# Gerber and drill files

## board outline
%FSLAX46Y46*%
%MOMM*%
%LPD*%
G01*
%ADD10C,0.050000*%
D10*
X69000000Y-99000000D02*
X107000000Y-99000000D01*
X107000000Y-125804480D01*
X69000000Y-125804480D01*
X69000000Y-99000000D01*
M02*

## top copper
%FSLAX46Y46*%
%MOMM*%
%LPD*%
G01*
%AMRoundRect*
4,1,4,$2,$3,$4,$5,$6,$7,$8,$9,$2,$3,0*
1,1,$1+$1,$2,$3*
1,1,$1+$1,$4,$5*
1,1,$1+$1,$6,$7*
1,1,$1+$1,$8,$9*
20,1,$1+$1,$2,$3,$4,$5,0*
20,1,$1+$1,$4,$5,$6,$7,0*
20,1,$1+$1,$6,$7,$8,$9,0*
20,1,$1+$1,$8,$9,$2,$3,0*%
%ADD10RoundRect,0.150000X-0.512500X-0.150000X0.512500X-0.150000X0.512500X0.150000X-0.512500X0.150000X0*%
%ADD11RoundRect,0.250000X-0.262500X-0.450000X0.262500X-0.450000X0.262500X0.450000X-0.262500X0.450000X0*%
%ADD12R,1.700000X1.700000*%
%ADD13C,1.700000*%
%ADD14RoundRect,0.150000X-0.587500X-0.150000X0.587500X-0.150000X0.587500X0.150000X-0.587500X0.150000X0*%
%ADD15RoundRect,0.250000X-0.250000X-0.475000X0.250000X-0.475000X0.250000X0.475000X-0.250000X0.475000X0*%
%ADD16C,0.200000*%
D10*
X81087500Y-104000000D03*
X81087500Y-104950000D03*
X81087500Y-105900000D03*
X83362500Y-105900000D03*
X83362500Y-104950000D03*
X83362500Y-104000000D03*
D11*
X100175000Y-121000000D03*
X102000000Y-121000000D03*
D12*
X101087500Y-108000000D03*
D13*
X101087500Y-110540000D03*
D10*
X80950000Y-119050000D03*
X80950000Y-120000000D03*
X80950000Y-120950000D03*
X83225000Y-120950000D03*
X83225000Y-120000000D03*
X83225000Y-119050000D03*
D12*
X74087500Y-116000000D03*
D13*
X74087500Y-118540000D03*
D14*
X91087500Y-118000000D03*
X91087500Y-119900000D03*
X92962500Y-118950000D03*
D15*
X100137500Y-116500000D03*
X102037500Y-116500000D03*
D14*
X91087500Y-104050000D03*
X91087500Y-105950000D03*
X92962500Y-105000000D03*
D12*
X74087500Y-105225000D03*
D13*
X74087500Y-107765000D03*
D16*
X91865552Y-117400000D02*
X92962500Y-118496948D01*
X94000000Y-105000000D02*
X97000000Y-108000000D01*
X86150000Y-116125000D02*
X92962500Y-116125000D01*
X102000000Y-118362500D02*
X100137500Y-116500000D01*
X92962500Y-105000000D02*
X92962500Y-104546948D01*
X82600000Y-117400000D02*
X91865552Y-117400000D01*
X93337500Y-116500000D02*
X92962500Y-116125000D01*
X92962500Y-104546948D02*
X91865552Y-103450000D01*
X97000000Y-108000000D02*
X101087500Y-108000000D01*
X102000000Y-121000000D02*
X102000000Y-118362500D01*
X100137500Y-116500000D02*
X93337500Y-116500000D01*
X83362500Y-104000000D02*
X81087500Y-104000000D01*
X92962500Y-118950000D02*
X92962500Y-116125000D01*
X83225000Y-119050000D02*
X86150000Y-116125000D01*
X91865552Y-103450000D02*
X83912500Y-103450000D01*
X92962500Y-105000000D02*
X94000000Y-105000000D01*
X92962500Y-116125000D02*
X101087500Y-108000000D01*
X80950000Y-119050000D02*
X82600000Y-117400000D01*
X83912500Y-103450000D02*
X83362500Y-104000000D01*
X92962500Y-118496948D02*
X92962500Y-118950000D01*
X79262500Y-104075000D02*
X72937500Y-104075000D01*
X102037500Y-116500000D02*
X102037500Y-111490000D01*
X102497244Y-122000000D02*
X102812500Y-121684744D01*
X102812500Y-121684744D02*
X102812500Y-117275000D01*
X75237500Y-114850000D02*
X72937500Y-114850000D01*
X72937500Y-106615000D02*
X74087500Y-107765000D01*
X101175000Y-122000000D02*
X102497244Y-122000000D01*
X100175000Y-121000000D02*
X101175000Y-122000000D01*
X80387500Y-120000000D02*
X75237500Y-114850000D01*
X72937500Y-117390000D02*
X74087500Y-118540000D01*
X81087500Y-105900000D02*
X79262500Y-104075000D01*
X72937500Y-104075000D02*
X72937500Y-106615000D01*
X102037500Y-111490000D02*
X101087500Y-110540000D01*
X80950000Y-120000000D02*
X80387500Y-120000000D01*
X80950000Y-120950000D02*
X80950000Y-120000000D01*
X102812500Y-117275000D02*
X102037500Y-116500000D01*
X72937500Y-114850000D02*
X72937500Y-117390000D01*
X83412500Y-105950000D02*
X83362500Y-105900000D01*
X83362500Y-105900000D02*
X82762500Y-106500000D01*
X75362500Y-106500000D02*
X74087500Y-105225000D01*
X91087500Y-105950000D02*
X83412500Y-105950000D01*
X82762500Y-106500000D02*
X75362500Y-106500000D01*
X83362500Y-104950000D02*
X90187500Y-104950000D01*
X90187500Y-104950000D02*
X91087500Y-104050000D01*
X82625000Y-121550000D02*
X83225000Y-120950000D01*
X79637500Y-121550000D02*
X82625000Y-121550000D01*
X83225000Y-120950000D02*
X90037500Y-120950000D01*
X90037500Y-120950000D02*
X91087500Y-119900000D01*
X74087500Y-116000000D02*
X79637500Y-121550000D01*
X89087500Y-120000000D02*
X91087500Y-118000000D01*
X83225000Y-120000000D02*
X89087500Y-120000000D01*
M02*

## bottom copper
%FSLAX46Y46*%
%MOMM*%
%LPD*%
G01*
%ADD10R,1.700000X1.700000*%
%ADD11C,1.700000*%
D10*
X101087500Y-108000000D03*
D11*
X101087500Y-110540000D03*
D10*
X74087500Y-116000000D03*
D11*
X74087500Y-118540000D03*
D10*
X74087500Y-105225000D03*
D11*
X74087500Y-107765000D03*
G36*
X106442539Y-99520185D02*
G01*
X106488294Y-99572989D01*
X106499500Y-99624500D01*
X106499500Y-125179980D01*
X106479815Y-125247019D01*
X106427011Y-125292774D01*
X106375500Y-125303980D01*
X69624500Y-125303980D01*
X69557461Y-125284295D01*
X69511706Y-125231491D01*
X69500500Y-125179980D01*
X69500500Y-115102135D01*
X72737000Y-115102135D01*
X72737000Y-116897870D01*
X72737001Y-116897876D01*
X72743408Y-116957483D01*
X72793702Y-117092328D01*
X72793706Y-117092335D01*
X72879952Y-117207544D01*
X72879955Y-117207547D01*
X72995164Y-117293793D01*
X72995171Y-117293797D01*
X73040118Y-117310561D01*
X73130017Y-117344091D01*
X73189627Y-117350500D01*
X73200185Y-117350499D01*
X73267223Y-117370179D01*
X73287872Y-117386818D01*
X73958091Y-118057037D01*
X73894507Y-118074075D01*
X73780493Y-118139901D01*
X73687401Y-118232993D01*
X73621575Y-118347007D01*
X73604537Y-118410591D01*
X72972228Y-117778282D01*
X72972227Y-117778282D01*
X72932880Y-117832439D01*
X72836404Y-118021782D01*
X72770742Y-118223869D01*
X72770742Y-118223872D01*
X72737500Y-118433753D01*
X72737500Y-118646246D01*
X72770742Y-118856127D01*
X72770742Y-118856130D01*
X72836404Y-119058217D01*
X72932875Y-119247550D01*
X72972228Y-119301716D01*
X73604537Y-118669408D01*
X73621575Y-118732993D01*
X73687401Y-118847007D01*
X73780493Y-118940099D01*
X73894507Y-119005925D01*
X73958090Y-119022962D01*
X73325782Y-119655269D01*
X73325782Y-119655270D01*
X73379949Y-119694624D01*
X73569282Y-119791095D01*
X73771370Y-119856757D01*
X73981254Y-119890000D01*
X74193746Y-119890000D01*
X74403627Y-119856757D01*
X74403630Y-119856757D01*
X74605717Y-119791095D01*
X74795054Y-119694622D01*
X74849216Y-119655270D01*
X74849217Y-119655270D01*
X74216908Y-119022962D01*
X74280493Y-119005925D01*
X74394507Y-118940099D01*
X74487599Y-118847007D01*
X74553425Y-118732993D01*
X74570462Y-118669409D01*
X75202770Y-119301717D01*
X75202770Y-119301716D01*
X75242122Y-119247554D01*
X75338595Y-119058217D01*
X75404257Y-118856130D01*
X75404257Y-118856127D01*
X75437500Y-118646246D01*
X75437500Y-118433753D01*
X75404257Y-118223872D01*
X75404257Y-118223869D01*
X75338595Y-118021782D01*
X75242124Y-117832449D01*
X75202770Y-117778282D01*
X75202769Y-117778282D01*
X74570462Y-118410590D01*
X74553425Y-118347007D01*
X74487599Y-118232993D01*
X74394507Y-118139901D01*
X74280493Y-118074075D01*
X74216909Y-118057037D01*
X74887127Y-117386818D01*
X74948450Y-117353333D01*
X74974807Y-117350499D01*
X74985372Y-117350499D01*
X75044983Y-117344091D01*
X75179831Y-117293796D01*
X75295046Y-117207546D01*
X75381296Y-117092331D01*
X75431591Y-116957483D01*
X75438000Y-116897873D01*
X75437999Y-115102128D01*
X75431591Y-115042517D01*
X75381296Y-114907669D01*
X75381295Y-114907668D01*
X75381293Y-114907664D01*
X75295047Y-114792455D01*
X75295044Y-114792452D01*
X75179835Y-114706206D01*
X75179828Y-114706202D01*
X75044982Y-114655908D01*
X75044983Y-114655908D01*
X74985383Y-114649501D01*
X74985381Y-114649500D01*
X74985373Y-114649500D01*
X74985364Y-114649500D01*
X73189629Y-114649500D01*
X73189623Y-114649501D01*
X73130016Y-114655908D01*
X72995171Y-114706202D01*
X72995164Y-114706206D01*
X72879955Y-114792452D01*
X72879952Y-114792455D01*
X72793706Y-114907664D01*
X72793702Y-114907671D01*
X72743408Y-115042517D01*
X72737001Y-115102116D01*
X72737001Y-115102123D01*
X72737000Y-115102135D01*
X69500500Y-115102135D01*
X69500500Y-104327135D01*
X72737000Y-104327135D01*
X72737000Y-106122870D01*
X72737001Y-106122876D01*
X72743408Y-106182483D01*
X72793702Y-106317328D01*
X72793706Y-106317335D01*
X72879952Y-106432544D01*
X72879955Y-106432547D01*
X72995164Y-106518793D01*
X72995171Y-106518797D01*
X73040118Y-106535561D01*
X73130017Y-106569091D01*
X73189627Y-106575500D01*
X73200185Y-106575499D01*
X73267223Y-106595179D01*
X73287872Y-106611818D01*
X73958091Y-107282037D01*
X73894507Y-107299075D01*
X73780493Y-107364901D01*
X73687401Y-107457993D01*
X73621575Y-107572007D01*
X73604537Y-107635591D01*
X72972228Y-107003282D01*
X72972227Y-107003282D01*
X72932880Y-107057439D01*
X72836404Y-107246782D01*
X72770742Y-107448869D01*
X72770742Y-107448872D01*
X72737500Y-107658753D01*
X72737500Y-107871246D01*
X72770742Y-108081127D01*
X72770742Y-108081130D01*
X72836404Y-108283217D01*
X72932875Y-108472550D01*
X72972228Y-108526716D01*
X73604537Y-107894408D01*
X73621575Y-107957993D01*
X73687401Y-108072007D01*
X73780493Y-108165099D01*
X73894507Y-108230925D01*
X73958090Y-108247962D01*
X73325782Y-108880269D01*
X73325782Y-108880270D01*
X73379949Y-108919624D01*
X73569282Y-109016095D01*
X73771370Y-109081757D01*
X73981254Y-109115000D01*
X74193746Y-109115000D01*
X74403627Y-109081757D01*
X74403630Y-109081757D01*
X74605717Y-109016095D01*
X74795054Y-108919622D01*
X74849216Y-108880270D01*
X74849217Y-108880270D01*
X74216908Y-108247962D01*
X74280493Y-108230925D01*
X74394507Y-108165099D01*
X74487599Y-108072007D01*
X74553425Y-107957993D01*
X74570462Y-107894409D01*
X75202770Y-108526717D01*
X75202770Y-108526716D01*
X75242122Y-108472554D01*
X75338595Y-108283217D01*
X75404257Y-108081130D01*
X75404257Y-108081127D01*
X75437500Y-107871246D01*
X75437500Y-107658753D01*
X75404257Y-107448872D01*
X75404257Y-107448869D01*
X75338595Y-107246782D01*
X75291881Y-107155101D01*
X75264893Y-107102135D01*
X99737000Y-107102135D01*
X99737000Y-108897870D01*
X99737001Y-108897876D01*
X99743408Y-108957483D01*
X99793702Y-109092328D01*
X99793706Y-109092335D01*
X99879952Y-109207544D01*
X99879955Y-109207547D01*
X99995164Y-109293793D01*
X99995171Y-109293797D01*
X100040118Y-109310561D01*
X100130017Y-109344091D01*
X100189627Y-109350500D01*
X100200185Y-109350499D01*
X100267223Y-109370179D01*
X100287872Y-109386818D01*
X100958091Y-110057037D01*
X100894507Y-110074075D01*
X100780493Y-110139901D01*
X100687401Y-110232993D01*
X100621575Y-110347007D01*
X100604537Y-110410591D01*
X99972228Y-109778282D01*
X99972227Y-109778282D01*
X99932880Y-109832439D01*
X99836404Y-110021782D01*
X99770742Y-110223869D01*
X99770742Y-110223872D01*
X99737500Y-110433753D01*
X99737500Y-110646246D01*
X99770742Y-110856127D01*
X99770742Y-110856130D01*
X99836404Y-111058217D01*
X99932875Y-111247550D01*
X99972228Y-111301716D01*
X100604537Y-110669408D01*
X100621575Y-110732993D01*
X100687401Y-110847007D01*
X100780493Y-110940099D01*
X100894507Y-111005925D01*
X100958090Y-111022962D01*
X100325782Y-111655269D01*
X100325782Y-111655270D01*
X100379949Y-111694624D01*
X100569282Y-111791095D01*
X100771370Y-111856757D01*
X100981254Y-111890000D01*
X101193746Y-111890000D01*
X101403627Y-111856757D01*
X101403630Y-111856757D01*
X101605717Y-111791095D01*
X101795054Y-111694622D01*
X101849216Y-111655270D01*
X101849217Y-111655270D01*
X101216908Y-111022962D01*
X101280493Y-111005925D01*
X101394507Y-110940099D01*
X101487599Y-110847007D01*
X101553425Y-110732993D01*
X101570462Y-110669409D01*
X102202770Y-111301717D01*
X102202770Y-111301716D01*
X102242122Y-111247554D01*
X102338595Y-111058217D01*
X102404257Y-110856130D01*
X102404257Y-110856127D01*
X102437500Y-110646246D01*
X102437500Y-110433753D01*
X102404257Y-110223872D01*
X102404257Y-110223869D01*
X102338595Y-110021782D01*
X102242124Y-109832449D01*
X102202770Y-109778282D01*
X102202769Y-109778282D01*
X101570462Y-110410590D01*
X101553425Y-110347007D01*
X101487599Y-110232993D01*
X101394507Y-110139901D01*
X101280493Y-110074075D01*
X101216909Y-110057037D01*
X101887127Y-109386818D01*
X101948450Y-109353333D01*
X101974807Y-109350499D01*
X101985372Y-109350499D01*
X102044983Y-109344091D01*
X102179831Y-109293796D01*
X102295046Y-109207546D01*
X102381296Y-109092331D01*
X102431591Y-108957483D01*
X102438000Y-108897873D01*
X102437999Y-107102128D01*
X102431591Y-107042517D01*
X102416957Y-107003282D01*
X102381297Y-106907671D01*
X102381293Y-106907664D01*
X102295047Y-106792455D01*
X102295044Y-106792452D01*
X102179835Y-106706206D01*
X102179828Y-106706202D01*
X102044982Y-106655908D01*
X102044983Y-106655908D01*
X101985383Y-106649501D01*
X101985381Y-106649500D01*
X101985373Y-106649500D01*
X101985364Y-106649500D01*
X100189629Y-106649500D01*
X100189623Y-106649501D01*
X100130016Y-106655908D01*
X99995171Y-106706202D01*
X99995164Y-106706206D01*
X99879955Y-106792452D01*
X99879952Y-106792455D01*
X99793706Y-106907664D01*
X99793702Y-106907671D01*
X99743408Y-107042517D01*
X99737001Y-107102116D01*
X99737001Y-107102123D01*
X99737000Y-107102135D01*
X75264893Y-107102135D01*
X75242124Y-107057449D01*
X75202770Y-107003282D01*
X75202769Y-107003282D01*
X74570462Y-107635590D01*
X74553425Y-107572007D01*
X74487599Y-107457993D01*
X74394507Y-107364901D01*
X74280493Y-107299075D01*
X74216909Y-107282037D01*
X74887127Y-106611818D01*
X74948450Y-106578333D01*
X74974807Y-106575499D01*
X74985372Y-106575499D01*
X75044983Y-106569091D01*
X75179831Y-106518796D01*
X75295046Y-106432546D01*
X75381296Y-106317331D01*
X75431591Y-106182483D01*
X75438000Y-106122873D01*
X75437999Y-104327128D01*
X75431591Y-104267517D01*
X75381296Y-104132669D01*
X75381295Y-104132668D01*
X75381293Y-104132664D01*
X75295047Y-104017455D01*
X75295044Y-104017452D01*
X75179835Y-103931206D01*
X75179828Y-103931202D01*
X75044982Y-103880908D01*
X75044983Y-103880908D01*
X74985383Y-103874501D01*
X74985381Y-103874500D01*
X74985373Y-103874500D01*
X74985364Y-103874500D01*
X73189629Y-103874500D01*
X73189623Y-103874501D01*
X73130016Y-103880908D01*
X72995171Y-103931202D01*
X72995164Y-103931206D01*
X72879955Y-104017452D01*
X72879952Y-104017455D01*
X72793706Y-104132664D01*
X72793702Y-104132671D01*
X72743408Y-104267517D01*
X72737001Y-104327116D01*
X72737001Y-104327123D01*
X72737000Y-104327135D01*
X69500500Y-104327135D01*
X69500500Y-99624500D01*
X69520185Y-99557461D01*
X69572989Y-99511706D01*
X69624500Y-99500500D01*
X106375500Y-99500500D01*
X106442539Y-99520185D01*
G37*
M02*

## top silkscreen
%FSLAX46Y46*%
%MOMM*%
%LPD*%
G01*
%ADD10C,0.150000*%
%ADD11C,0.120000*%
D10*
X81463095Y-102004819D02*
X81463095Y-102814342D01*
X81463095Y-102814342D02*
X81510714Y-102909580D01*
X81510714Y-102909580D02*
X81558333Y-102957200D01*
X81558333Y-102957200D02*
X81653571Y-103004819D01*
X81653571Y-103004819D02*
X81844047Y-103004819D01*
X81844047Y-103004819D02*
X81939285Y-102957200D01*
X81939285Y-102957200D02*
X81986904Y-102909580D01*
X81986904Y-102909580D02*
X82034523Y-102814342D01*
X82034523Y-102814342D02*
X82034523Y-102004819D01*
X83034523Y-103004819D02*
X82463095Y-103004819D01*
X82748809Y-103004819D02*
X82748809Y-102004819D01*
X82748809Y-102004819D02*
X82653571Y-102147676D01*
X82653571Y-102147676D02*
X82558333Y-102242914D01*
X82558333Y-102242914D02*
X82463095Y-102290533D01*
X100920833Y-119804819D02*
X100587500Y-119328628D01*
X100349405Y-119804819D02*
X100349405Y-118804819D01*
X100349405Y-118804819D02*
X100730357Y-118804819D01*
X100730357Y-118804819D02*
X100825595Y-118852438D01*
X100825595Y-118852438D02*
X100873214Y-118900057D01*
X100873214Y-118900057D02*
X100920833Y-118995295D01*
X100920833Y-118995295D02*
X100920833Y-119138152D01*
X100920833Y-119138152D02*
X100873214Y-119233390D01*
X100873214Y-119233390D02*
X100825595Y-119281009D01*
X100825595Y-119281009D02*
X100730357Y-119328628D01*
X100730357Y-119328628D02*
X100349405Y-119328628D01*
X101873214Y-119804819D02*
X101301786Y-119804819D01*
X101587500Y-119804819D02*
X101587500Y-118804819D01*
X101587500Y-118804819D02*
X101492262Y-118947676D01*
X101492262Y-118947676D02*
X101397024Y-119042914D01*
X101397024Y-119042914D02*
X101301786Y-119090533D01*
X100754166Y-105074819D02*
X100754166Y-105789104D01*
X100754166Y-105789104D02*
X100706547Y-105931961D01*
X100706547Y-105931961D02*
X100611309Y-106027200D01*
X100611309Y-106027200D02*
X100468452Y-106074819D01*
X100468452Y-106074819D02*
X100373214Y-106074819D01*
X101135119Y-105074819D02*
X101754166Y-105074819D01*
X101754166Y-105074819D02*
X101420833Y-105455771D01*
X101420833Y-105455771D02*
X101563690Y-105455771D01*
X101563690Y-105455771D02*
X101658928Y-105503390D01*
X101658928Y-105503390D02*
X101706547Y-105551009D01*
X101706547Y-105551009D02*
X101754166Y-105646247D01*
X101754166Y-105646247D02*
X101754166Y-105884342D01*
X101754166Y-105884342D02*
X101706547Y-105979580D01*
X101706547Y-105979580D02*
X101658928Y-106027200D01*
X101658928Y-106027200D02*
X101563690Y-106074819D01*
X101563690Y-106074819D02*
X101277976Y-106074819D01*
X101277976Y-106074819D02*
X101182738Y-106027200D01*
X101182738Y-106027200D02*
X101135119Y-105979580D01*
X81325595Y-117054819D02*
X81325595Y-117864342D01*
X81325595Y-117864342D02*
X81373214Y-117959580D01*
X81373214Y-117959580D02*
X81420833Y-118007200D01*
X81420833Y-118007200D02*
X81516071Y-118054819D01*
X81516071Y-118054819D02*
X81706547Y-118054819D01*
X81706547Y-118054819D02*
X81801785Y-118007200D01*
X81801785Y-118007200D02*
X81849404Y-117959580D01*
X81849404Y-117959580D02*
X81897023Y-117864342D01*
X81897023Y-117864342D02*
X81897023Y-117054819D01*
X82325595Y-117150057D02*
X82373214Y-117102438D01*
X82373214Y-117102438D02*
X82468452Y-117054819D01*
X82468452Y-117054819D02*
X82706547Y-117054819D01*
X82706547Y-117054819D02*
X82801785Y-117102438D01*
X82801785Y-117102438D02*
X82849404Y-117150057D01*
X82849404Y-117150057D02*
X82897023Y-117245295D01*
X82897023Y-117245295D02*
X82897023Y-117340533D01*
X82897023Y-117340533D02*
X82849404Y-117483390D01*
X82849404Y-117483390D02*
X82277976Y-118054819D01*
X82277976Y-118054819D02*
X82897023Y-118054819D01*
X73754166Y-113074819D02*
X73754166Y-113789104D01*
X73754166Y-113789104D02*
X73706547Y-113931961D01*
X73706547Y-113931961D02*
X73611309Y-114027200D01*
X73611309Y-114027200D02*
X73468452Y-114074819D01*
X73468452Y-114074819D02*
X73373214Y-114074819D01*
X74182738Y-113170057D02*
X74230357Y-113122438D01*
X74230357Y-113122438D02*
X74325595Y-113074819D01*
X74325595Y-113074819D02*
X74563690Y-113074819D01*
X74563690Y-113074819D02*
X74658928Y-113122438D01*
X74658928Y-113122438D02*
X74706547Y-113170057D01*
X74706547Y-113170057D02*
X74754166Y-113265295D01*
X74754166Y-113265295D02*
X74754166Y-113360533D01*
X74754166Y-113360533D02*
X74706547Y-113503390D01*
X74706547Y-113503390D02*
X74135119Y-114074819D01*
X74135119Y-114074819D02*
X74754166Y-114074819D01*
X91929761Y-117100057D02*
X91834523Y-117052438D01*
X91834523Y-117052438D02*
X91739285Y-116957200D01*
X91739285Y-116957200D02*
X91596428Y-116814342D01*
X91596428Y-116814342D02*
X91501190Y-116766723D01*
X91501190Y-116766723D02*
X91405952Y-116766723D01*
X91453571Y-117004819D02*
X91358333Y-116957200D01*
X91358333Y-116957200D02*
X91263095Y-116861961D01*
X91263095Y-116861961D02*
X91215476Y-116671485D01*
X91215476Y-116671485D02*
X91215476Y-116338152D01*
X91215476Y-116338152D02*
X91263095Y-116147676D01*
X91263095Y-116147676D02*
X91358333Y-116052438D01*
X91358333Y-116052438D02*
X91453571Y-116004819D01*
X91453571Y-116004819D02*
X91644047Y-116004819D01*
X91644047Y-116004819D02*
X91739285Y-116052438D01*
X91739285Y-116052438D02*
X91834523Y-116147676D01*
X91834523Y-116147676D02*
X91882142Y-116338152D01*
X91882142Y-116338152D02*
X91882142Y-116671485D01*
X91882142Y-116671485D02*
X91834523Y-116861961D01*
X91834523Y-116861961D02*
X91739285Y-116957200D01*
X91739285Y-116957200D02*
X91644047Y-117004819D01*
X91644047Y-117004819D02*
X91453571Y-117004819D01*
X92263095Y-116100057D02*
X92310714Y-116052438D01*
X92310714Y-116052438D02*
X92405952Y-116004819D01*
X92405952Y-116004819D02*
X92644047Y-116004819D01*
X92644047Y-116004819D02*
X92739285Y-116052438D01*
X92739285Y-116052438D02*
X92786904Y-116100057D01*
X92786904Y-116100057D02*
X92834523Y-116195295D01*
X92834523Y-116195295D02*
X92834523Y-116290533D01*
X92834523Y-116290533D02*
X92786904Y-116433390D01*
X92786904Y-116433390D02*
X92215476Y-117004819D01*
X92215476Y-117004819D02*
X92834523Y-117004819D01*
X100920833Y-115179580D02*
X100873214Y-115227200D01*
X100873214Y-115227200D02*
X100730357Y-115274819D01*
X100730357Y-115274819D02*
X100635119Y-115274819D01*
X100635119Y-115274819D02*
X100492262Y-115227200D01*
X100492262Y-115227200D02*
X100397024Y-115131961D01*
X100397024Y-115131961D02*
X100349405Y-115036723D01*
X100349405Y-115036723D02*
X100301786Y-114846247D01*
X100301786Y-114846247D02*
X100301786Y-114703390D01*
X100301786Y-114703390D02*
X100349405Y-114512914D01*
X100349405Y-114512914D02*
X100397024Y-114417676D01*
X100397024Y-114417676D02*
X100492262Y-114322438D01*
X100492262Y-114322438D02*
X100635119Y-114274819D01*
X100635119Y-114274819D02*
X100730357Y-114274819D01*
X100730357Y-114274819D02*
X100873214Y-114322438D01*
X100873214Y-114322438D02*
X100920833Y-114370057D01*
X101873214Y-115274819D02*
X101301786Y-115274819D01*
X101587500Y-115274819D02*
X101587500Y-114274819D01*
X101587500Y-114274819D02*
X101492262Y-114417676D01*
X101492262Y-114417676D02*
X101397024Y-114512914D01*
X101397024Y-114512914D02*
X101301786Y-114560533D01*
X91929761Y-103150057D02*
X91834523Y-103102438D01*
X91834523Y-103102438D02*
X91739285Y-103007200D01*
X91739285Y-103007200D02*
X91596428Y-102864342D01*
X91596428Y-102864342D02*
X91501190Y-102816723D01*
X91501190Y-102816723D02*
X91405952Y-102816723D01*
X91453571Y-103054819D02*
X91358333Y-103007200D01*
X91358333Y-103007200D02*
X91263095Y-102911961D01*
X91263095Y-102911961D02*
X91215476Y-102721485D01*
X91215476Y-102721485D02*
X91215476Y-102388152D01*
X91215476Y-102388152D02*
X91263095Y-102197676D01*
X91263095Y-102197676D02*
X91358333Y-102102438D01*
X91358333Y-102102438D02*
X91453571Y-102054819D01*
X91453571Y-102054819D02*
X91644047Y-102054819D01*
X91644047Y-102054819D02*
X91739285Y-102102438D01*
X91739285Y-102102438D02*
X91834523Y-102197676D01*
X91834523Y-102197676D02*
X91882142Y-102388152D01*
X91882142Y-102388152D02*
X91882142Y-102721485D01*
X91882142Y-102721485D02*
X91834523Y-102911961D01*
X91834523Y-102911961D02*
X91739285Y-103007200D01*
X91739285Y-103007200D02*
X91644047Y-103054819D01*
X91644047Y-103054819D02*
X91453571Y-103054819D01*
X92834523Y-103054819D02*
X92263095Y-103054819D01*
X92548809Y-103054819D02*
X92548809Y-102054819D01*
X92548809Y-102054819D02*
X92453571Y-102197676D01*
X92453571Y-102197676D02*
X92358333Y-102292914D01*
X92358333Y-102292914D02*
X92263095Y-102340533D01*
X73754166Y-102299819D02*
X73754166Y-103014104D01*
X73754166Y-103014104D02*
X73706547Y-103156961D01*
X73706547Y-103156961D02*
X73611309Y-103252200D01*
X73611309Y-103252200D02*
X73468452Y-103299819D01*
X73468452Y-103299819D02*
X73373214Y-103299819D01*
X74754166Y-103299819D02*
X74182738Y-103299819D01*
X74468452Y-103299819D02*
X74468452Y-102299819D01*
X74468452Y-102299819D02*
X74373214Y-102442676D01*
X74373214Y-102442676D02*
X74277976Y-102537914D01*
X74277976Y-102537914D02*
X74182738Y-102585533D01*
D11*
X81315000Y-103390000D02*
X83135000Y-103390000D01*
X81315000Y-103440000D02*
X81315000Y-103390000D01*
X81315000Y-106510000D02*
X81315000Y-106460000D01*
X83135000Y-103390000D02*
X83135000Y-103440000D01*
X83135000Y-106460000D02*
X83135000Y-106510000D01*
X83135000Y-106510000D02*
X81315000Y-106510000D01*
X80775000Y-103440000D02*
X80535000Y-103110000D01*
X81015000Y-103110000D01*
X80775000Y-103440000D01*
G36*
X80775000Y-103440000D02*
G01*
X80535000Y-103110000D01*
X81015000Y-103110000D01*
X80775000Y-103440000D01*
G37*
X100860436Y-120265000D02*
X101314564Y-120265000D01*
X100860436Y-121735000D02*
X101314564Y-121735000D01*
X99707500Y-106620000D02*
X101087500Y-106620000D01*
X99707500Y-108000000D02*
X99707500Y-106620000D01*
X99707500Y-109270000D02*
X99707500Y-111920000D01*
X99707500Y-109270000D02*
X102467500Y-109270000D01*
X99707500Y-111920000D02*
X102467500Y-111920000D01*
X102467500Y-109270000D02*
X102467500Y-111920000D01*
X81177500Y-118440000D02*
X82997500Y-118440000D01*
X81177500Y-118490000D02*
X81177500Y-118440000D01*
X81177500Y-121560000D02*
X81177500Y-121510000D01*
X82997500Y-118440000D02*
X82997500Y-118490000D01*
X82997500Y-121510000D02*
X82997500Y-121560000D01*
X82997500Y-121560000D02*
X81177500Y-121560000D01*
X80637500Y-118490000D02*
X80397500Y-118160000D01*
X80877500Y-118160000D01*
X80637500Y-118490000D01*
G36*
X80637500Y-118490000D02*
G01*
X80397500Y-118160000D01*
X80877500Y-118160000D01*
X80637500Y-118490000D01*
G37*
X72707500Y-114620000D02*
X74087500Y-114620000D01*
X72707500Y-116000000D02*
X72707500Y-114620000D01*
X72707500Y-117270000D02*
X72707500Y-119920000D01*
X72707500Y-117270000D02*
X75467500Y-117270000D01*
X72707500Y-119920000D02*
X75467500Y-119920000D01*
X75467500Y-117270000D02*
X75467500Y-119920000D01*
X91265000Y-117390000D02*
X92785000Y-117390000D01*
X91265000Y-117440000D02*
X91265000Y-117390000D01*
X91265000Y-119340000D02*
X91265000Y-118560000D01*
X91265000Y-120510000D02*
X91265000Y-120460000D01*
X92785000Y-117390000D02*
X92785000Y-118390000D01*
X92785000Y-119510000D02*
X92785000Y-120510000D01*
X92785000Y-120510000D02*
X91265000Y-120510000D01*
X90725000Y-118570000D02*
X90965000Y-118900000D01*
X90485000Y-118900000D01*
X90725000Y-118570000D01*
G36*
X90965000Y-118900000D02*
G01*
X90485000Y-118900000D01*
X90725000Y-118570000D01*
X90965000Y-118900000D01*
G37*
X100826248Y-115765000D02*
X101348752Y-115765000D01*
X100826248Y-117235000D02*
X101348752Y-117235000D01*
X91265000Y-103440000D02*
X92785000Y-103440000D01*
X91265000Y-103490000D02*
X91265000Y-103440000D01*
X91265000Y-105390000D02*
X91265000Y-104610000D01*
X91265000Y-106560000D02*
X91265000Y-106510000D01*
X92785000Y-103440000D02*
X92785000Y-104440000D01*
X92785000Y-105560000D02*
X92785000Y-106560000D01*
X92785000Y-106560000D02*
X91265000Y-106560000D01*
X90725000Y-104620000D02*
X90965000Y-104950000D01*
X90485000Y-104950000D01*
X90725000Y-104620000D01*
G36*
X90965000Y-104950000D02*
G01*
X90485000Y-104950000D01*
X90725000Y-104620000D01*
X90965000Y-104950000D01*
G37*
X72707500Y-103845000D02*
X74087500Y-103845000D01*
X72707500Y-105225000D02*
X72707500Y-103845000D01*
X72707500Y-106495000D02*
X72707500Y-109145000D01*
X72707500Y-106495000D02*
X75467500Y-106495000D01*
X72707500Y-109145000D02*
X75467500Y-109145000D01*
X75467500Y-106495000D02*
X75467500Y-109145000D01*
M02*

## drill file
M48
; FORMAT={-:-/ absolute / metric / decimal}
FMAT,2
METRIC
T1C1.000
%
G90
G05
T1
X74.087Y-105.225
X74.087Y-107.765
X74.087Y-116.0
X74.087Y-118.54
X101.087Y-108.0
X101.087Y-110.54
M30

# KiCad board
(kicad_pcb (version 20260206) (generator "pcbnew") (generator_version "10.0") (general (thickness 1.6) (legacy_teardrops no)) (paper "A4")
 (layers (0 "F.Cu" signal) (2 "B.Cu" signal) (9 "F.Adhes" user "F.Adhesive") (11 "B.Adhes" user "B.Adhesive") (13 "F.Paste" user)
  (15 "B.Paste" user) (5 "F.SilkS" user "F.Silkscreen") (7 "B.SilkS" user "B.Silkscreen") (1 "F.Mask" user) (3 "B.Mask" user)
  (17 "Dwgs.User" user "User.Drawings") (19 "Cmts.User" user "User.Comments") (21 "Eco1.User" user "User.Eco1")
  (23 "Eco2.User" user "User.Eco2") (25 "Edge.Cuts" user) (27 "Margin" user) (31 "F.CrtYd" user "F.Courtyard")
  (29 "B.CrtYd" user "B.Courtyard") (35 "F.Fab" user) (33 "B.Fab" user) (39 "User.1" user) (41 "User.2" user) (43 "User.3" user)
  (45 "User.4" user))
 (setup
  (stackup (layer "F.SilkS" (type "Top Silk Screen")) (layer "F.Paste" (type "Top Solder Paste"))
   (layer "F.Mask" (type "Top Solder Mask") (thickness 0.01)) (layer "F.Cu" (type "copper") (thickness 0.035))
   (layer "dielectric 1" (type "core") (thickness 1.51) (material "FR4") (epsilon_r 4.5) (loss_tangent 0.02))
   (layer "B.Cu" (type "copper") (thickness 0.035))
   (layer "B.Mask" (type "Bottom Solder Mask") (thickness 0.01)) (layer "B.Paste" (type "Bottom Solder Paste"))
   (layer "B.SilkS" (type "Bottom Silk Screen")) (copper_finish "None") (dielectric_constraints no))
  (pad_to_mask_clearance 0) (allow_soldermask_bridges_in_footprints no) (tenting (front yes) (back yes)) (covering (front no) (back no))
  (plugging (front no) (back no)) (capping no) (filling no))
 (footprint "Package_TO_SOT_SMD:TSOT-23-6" (layer "F.Cu") (at 82.225 104.95)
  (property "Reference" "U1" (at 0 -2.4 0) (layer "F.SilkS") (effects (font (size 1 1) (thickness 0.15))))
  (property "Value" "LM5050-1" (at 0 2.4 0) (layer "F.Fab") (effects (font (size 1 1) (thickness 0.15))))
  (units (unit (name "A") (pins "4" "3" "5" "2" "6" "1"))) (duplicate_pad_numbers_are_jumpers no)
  (fp_line (start -0.91 -1.56) (end 0.91 -1.56) (stroke (width 0.12) (type solid)) (layer "F.SilkS"))
  (fp_line (start -0.91 -1.51) (end -0.91 -1.56) (stroke (width 0.12) (type solid)) (layer "F.SilkS"))
  (fp_line (start -0.91 1.56) (end -0.91 1.51) (stroke (width 0.12) (type solid)) (layer "F.SilkS"))
  (fp_line (start 0.91 -1.56) (end 0.91 -1.51) (stroke (width 0.12) (type solid)) (layer "F.SilkS"))
  (fp_line (start 0.91 1.51) (end 0.91 1.56) (stroke (width 0.12) (type solid)) (layer "F.SilkS"))
  (fp_line (start 0.91 1.56) (end -0.91 1.56) (stroke (width 0.12) (type solid)) (layer "F.SilkS"))
  (fp_poly (pts (xy -1.45 -1.51) (xy -1.69 -1.84) (xy -1.21 -1.84)) (stroke (width 0.12) (type solid)) (fill yes) (layer "F.SilkS"))
  (pad "1" smd roundrect (at -1.1375 -0.95) (size 1.325 0.6) (layers "F.Cu" "F.Mask" "F.Paste") (roundrect_rratio 0.25)
   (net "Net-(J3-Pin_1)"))
  (pad "2" smd roundrect (at -1.1375 0) (size 1.325 0.6) (layers "F.Cu" "F.Mask" "F.Paste") (roundrect_rratio 0.25) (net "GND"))
  (pad "3" smd roundrect (at -1.1375 0.95) (size 1.325 0.6) (layers "F.Cu" "F.Mask" "F.Paste") (roundrect_rratio 0.25) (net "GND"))
  (pad "4" smd roundrect (at 1.1375 0.95) (size 1.325 0.6) (layers "F.Cu" "F.Mask" "F.Paste") (roundrect_rratio 0.25) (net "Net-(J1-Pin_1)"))
  (pad "5" smd roundrect (at 1.1375 0) (size 1.325 0.6) (layers "F.Cu" "F.Mask" "F.Paste") (roundrect_rratio 0.25) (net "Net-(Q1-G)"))
  (pad "6" smd roundrect (at 1.1375 -0.95) (size 1.325 0.6) (layers "F.Cu" "F.Mask" "F.Paste") (roundrect_rratio 0.25)
   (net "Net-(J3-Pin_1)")))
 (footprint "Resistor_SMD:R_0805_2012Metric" (layer "F.Cu") (at 101.0875 121)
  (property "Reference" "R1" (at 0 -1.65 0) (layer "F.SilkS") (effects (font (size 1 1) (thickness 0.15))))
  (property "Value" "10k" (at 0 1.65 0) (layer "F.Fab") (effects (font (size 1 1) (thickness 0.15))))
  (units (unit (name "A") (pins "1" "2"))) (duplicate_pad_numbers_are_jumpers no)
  (fp_line (start -0.227064 -0.735) (end 0.227064 -0.735) (stroke (width 0.12) (type solid)) (layer "F.SilkS"))
  (fp_line (start -0.227064 0.735) (end 0.227064 0.735) (stroke (width 0.12) (type solid)) (layer "F.SilkS"))
  (pad "1" smd roundrect (at -0.9125 0) (size 1.025 1.4) (layers "F.Cu" "F.Mask" "F.Paste") (roundrect_rratio 0.243902) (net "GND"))
  (pad "2" smd roundrect (at 0.9125 0) (size 1.025 1.4) (layers "F.Cu" "F.Mask" "F.Paste") (roundrect_rratio 0.243902)
   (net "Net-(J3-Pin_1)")))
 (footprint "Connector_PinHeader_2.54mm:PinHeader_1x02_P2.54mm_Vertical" (layer "F.Cu") (at 101.0875 108)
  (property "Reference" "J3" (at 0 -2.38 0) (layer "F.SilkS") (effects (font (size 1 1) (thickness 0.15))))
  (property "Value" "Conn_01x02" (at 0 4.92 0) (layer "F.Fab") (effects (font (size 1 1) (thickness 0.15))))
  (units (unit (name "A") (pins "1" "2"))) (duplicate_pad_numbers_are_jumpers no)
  (fp_line (start -1.38 -1.38) (end 0 -1.38) (stroke (width 0.12) (type solid)) (layer "F.SilkS"))
  (fp_line (start -1.38 0) (end -1.38 -1.38) (stroke (width 0.12) (type solid)) (layer "F.SilkS"))
  (fp_line (start -1.38 1.27) (end -1.38 3.92) (stroke (width 0.12) (type solid)) (layer "F.SilkS"))
  (fp_line (start -1.38 1.27) (end 1.38 1.27) (stroke (width 0.12) (type solid)) (layer "F.SilkS"))
  (fp_line (start -1.38 3.92) (end 1.38 3.92) (stroke (width 0.12) (type solid)) (layer "F.SilkS"))
  (fp_line (start 1.38 1.27) (end 1.38 3.92) (stroke (width 0.12) (type solid)) (layer "F.SilkS"))
  (pad "1" thru_hole rect (at 0 0) (size 1.7 1.7) (drill 1) (layers "*.Cu" "*.Mask") (remove_unused_layers no) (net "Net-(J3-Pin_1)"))
  (pad "2" thru_hole circle (at 0 2.54) (size 1.7 1.7) (drill 1) (layers "*.Cu" "*.Mask") (remove_unused_layers no) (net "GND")))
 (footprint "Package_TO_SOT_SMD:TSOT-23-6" (layer "F.Cu") (at 82.0875 120)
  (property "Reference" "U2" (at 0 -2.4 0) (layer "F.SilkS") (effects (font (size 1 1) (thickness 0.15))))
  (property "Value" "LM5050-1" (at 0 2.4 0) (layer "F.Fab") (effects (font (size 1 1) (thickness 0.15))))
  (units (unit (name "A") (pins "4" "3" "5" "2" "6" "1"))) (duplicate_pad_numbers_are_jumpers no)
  (fp_line (start -0.91 -1.56) (end 0.91 -1.56) (stroke (width 0.12) (type solid)) (layer "F.SilkS"))
  (fp_line (start -0.91 -1.51) (end -0.91 -1.56) (stroke (width 0.12) (type solid)) (layer "F.SilkS"))
  (fp_line (start -0.91 1.56) (end -0.91 1.51) (stroke (width 0.12) (type solid)) (layer "F.SilkS"))
  (fp_line (start 0.91 -1.56) (end 0.91 -1.51) (stroke (width 0.12) (type solid)) (layer "F.SilkS"))
  (fp_line (start 0.91 1.51) (end 0.91 1.56) (stroke (width 0.12) (type solid)) (layer "F.SilkS"))
  (fp_line (start 0.91 1.56) (end -0.91 1.56) (stroke (width 0.12) (type solid)) (layer "F.SilkS"))
  (fp_poly (pts (xy -1.45 -1.51) (xy -1.69 -1.84) (xy -1.21 -1.84)) (stroke (width 0.12) (type solid)) (fill yes) (layer "F.SilkS"))
  (pad "1" smd roundrect (at -1.1375 -0.95) (size 1.325 0.6) (layers "F.Cu" "F.Mask" "F.Paste") (roundrect_rratio 0.25)
   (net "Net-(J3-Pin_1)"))
  (pad "2" smd roundrect (at -1.1375 0) (size 1.325 0.6) (layers "F.Cu" "F.Mask" "F.Paste") (roundrect_rratio 0.25) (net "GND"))
  (pad "3" smd roundrect (at -1.1375 0.95) (size 1.325 0.6) (layers "F.Cu" "F.Mask" "F.Paste") (roundrect_rratio 0.25) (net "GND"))
  (pad "4" smd roundrect (at 1.1375 0.95) (size 1.325 0.6) (layers "F.Cu" "F.Mask" "F.Paste") (roundrect_rratio 0.25) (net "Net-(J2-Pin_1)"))
  (pad "5" smd roundrect (at 1.1375 0) (size 1.325 0.6) (layers "F.Cu" "F.Mask" "F.Paste") (roundrect_rratio 0.25) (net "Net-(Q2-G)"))
  (pad "6" smd roundrect (at 1.1375 -0.95) (size 1.325 0.6) (layers "F.Cu" "F.Mask" "F.Paste") (roundrect_rratio 0.25)
   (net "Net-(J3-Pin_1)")))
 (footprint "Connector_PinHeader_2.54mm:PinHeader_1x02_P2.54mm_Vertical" (layer "F.Cu") (at 74.0875 116)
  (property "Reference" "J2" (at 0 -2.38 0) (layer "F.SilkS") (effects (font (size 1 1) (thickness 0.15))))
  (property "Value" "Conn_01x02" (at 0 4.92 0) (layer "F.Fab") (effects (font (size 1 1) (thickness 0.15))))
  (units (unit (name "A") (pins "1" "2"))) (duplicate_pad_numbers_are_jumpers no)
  (fp_line (start -1.38 -1.38) (end 0 -1.38) (stroke (width 0.12) (type solid)) (layer "F.SilkS"))
  (fp_line (start -1.38 0) (end -1.38 -1.38) (stroke (width 0.12) (type solid)) (layer "F.SilkS"))
  (fp_line (start -1.38 1.27) (end -1.38 3.92) (stroke (width 0.12) (type solid)) (layer "F.SilkS"))
  (fp_line (start -1.38 1.27) (end 1.38 1.27) (stroke (width 0.12) (type solid)) (layer "F.SilkS"))
  (fp_line (start -1.38 3.92) (end 1.38 3.92) (stroke (width 0.12) (type solid)) (layer "F.SilkS"))
  (fp_line (start 1.38 1.27) (end 1.38 3.92) (stroke (width 0.12) (type solid)) (layer "F.SilkS"))
  (pad "1" thru_hole rect (at 0 0) (size 1.7 1.7) (drill 1) (layers "*.Cu" "*.Mask") (remove_unused_layers no) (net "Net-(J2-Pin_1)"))
  (pad "2" thru_hole circle (at 0 2.54) (size 1.7 1.7) (drill 1) (layers "*.Cu" "*.Mask") (remove_unused_layers no) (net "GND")))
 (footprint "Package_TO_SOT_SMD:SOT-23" (layer "F.Cu") (at 92.025 118.95)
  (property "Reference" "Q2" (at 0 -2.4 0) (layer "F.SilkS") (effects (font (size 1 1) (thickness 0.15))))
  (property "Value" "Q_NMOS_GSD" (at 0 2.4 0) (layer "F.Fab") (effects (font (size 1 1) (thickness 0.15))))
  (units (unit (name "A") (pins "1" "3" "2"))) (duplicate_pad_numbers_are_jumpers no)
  (fp_line (start -0.76 -1.56) (end 0.76 -1.56) (stroke (width 0.12) (type solid)) (layer "F.SilkS"))
  (fp_line (start -0.76 -1.51) (end -0.76 -1.56) (stroke (width 0.12) (type solid)) (layer "F.SilkS"))
  (fp_line (start -0.76 0.39) (end -0.76 -0.39) (stroke (width 0.12) (type solid)) (layer "F.SilkS"))
  (fp_line (start -0.76 1.56) (end -0.76 1.51) (stroke (width 0.12) (type solid)) (layer "F.SilkS"))
  (fp_line (start 0.76 -1.56) (end 0.76 -0.56) (stroke (width 0.12) (type solid)) (layer "F.SilkS"))
  (fp_line (start 0.76 0.56) (end 0.76 1.56) (stroke (width 0.12) (type solid)) (layer "F.SilkS"))
  (fp_line (start 0.76 1.56) (end -0.76 1.56) (stroke (width 0.12) (type solid)) (layer "F.SilkS"))
  (fp_poly (pts (xy -1.3 -0.38) (xy -1.06 -0.05) (xy -1.54 -0.05)) (stroke (width 0.12) (type solid)) (fill yes) (layer "F.SilkS"))
  (pad "1" smd roundrect (at -0.9375 -0.95) (size 1.475 0.6) (layers "F.Cu" "F.Mask" "F.Paste") (roundrect_rratio 0.25) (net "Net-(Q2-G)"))
  (pad "2" smd roundrect (at -0.9375 0.95) (size 1.475 0.6) (layers "F.Cu" "F.Mask" "F.Paste") (roundrect_rratio 0.25)
   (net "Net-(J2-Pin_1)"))
  (pad "3" smd roundrect (at 0.9375 0) (size 1.475 0.6) (layers "F.Cu" "F.Mask" "F.Paste") (roundrect_rratio 0.25) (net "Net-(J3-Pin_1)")))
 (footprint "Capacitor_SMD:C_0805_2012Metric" (layer "F.Cu") (at 101.0875 116.5)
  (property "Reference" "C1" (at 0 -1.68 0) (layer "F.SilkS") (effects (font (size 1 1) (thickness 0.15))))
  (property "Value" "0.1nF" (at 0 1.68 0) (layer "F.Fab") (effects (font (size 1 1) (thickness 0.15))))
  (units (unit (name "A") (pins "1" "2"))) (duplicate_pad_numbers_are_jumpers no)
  (fp_line (start -0.261252 -0.735) (end 0.261252 -0.735) (stroke (width 0.12) (type solid)) (layer "F.SilkS"))
  (fp_line (start -0.261252 0.735) (end 0.261252 0.735) (stroke (width 0.12) (type solid)) (layer "F.SilkS"))
  (pad "1" smd roundrect (at -0.95 0) (size 1 1.45) (layers "F.Cu" "F.Mask" "F.Paste") (roundrect_rratio 0.25) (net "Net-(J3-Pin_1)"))
  (pad "2" smd roundrect (at 0.95 0) (size 1 1.45) (layers "F.Cu" "F.Mask" "F.Paste") (roundrect_rratio 0.25) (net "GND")))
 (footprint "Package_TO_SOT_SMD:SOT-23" (layer "F.Cu") (at 92.025 105)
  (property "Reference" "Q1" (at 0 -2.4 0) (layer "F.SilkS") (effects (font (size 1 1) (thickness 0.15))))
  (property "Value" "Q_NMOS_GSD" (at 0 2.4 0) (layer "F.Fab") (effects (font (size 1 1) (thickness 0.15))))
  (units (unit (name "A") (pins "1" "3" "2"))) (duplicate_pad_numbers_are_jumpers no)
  (fp_line (start -0.76 -1.56) (end 0.76 -1.56) (stroke (width 0.12) (type solid)) (layer "F.SilkS"))
  (fp_line (start -0.76 -1.51) (end -0.76 -1.56) (stroke (width 0.12) (type solid)) (layer "F.SilkS"))
  (fp_line (start -0.76 0.39) (end -0.76 -0.39) (stroke (width 0.12) (type solid)) (layer "F.SilkS"))
  (fp_line (start -0.76 1.56) (end -0.76 1.51) (stroke (width 0.12) (type solid)) (layer "F.SilkS"))
  (fp_line (start 0.76 -1.56) (end 0.76 -0.56) (stroke (width 0.12) (type solid)) (layer "F.SilkS"))
  (fp_line (start 0.76 0.56) (end 0.76 1.56) (stroke (width 0.12) (type solid)) (layer "F.SilkS"))
  (fp_line (start 0.76 1.56) (end -0.76 1.56) (stroke (width 0.12) (type solid)) (layer "F.SilkS"))
  (fp_poly (pts (xy -1.3 -0.38) (xy -1.06 -0.05) (xy -1.54 -0.05)) (stroke (width 0.12) (type solid)) (fill yes) (layer "F.SilkS"))
  (pad "1" smd roundrect (at -0.9375 -0.95) (size 1.475 0.6) (layers "F.Cu" "F.Mask" "F.Paste") (roundrect_rratio 0.25) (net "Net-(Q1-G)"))
  (pad "2" smd roundrect (at -0.9375 0.95) (size 1.475 0.6) (layers "F.Cu" "F.Mask" "F.Paste") (roundrect_rratio 0.25)
   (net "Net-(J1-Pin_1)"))
  (pad "3" smd roundrect (at 0.9375 0) (size 1.475 0.6) (layers "F.Cu" "F.Mask" "F.Paste") (roundrect_rratio 0.25) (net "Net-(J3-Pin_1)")))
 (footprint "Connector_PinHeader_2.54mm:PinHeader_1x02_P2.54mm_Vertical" (layer "F.Cu") (at 74.0875 105.225)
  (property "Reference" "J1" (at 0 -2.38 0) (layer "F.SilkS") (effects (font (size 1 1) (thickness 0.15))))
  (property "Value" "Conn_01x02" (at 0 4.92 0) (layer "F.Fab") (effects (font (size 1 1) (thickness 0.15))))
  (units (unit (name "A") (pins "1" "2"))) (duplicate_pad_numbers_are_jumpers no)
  (fp_line (start -1.38 -1.38) (end 0 -1.38) (stroke (width 0.12) (type solid)) (layer "F.SilkS"))
  (fp_line (start -1.38 0) (end -1.38 -1.38) (stroke (width 0.12) (type solid)) (layer "F.SilkS"))
  (fp_line (start -1.38 1.27) (end -1.38 3.92) (stroke (width 0.12) (type solid)) (layer "F.SilkS"))
  (fp_line (start -1.38 1.27) (end 1.38 1.27) (stroke (width 0.12) (type solid)) (layer "F.SilkS"))
  (fp_line (start -1.38 3.92) (end 1.38 3.92) (stroke (width 0.12) (type solid)) (layer "F.SilkS"))
  (fp_line (start 1.38 1.27) (end 1.38 3.92) (stroke (width 0.12) (type solid)) (layer "F.SilkS"))
  (pad "1" thru_hole rect (at 0 0) (size 1.7 1.7) (drill 1) (layers "*.Cu" "*.Mask") (remove_unused_layers no) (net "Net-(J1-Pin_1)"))
  (pad "2" thru_hole circle (at 0 2.54) (size 1.7 1.7) (drill 1) (layers "*.Cu" "*.Mask") (remove_unused_layers no) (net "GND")))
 (gr_rect (start 69 99) (end 107 125.80448) (stroke (width 0.05) (type default)) (fill no) (layer "Edge.Cuts"))
 (segment (start 91.865552 117.4) (end 92.9625 118.496948) (width 0.2) (layer "F.Cu") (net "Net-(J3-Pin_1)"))
 (segment (start 94 105) (end 97 108) (width 0.2) (layer "F.Cu") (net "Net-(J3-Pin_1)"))
 (segment (start 86.15 116.125) (end 92.9625 116.125) (width 0.2) (layer "F.Cu") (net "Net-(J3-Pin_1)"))
 (segment (start 102 118.3625) (end 100.1375 116.5) (width 0.2) (layer "F.Cu") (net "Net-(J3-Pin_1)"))
 (segment (start 92.9625 105) (end 92.9625 104.546948) (width 0.2) (layer "F.Cu") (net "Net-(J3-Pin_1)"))
 (segment (start 82.6 117.4) (end 91.865552 117.4) (width 0.2) (layer "F.Cu") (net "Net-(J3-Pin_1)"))
 (segment (start 93.3375 116.5) (end 92.9625 116.125) (width 0.2) (layer "F.Cu") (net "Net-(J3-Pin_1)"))
 (segment (start 92.9625 104.546948) (end 91.865552 103.45) (width 0.2) (layer "F.Cu") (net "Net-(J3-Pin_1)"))
 (segment (start 97 108) (end 101.0875 108) (width 0.2) (layer "F.Cu") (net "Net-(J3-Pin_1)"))
 (segment (start 102 121) (end 102 118.3625) (width 0.2) (layer "F.Cu") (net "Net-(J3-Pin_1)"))
 (segment (start 100.1375 116.5) (end 93.3375 116.5) (width 0.2) (layer "F.Cu") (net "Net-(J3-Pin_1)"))
 (segment (start 83.3625 104) (end 81.0875 104) (width 0.2) (layer "F.Cu") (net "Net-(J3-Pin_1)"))
 (segment (start 92.9625 118.95) (end 92.9625 116.125) (width 0.2) (layer "F.Cu") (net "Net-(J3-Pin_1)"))
 (segment (start 83.225 119.05) (end 86.15 116.125) (width 0.2) (layer "F.Cu") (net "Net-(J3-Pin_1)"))
 (segment (start 91.865552 103.45) (end 83.9125 103.45) (width 0.2) (layer "F.Cu") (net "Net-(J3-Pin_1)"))
 (segment (start 92.9625 105) (end 94 105) (width 0.2) (layer "F.Cu") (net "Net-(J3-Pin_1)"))
 (segment (start 92.9625 116.125) (end 101.0875 108) (width 0.2) (layer "F.Cu") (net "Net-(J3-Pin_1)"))
 (segment (start 80.95 119.05) (end 82.6 117.4) (width 0.2) (layer "F.Cu") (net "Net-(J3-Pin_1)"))
 (segment (start 83.9125 103.45) (end 83.3625 104) (width 0.2) (layer "F.Cu") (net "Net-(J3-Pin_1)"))
 (segment (start 92.9625 118.496948) (end 92.9625 118.95) (width 0.2) (layer "F.Cu") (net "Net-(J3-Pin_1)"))
 (segment (start 79.2625 104.075) (end 72.9375 104.075) (width 0.2) (layer "F.Cu") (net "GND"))
 (segment (start 102.0375 116.5) (end 102.0375 111.49) (width 0.2) (layer "F.Cu") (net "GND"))
 (segment (start 102.497244 122) (end 102.8125 121.684744) (width 0.2) (layer "F.Cu") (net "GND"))
 (segment (start 102.8125 121.684744) (end 102.8125 117.275) (width 0.2) (layer "F.Cu") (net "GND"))
 (segment (start 75.2375 114.85) (end 72.9375 114.85) (width 0.2) (layer "F.Cu") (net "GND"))
 (segment (start 72.9375 106.615) (end 74.0875 107.765) (width 0.2) (layer "F.Cu") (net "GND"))
 (segment (start 101.175 122) (end 102.497244 122) (width 0.2) (layer "F.Cu") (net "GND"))
 (segment (start 100.175 121) (end 101.175 122) (width 0.2) (layer "F.Cu") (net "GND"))
 (segment (start 80.3875 120) (end 75.2375 114.85) (width 0.2) (layer "F.Cu") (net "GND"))
 (segment (start 72.9375 117.39) (end 74.0875 118.54) (width 0.2) (layer "F.Cu") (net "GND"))
 (segment (start 81.0875 105.9) (end 79.2625 104.075) (width 0.2) (layer "F.Cu") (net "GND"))
 (segment (start 72.9375 104.075) (end 72.9375 106.615) (width 0.2) (layer "F.Cu") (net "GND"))
 (segment (start 102.0375 111.49) (end 101.0875 110.54) (width 0.2) (layer "F.Cu") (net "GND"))
 (segment (start 80.95 120) (end 80.3875 120) (width 0.2) (layer "F.Cu") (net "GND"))
 (segment (start 80.95 120.95) (end 80.95 120) (width 0.2) (layer "F.Cu") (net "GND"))
 (segment (start 102.8125 117.275) (end 102.0375 116.5) (width 0.2) (layer "F.Cu") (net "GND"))
 (segment (start 72.9375 114.85) (end 72.9375 117.39) (width 0.2) (layer "F.Cu") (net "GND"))
 (segment (start 83.4125 105.95) (end 83.3625 105.9) (width 0.2) (layer "F.Cu") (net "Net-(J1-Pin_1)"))
 (segment (start 83.3625 105.9) (end 82.7625 106.5) (width 0.2) (layer "F.Cu") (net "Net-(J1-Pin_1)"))
 (segment (start 75.3625 106.5) (end 74.0875 105.225) (width 0.2) (layer "F.Cu") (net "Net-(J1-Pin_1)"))
 (segment (start 91.0875 105.95) (end 83.4125 105.95) (width 0.2) (layer "F.Cu") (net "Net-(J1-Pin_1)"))
 (segment (start 82.7625 106.5) (end 75.3625 106.5) (width 0.2) (layer "F.Cu") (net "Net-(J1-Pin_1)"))
 (segment (start 83.3625 104.95) (end 90.1875 104.95) (width 0.2) (layer "F.Cu") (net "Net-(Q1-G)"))
 (segment (start 90.1875 104.95) (end 91.0875 104.05) (width 0.2) (layer "F.Cu") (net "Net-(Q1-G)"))
 (segment (start 82.625 121.55) (end 83.225 120.95) (width 0.2) (layer "F.Cu") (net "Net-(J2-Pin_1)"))
 (segment (start 79.6375 121.55) (end 82.625 121.55) (width 0.2) (layer "F.Cu") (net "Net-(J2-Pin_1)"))
 (segment (start 83.225 120.95) (end 90.0375 120.95) (width 0.2) (layer "F.Cu") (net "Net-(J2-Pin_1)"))
 (segment (start 90.0375 120.95) (end 91.0875 119.9) (width 0.2) (layer "F.Cu") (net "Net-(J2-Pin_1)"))
 (segment (start 74.0875 116) (end 79.6375 121.55) (width 0.2) (layer "F.Cu") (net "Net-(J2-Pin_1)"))
 (segment (start 89.0875 120) (end 91.0875 118) (width 0.2) (layer "F.Cu") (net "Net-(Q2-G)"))
 (segment (start 83.225 120) (end 89.0875 120) (width 0.2) (layer "F.Cu") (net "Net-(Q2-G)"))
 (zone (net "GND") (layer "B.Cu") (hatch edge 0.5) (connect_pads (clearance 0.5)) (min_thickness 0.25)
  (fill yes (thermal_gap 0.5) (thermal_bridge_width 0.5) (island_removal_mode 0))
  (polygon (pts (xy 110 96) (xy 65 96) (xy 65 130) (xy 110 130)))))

